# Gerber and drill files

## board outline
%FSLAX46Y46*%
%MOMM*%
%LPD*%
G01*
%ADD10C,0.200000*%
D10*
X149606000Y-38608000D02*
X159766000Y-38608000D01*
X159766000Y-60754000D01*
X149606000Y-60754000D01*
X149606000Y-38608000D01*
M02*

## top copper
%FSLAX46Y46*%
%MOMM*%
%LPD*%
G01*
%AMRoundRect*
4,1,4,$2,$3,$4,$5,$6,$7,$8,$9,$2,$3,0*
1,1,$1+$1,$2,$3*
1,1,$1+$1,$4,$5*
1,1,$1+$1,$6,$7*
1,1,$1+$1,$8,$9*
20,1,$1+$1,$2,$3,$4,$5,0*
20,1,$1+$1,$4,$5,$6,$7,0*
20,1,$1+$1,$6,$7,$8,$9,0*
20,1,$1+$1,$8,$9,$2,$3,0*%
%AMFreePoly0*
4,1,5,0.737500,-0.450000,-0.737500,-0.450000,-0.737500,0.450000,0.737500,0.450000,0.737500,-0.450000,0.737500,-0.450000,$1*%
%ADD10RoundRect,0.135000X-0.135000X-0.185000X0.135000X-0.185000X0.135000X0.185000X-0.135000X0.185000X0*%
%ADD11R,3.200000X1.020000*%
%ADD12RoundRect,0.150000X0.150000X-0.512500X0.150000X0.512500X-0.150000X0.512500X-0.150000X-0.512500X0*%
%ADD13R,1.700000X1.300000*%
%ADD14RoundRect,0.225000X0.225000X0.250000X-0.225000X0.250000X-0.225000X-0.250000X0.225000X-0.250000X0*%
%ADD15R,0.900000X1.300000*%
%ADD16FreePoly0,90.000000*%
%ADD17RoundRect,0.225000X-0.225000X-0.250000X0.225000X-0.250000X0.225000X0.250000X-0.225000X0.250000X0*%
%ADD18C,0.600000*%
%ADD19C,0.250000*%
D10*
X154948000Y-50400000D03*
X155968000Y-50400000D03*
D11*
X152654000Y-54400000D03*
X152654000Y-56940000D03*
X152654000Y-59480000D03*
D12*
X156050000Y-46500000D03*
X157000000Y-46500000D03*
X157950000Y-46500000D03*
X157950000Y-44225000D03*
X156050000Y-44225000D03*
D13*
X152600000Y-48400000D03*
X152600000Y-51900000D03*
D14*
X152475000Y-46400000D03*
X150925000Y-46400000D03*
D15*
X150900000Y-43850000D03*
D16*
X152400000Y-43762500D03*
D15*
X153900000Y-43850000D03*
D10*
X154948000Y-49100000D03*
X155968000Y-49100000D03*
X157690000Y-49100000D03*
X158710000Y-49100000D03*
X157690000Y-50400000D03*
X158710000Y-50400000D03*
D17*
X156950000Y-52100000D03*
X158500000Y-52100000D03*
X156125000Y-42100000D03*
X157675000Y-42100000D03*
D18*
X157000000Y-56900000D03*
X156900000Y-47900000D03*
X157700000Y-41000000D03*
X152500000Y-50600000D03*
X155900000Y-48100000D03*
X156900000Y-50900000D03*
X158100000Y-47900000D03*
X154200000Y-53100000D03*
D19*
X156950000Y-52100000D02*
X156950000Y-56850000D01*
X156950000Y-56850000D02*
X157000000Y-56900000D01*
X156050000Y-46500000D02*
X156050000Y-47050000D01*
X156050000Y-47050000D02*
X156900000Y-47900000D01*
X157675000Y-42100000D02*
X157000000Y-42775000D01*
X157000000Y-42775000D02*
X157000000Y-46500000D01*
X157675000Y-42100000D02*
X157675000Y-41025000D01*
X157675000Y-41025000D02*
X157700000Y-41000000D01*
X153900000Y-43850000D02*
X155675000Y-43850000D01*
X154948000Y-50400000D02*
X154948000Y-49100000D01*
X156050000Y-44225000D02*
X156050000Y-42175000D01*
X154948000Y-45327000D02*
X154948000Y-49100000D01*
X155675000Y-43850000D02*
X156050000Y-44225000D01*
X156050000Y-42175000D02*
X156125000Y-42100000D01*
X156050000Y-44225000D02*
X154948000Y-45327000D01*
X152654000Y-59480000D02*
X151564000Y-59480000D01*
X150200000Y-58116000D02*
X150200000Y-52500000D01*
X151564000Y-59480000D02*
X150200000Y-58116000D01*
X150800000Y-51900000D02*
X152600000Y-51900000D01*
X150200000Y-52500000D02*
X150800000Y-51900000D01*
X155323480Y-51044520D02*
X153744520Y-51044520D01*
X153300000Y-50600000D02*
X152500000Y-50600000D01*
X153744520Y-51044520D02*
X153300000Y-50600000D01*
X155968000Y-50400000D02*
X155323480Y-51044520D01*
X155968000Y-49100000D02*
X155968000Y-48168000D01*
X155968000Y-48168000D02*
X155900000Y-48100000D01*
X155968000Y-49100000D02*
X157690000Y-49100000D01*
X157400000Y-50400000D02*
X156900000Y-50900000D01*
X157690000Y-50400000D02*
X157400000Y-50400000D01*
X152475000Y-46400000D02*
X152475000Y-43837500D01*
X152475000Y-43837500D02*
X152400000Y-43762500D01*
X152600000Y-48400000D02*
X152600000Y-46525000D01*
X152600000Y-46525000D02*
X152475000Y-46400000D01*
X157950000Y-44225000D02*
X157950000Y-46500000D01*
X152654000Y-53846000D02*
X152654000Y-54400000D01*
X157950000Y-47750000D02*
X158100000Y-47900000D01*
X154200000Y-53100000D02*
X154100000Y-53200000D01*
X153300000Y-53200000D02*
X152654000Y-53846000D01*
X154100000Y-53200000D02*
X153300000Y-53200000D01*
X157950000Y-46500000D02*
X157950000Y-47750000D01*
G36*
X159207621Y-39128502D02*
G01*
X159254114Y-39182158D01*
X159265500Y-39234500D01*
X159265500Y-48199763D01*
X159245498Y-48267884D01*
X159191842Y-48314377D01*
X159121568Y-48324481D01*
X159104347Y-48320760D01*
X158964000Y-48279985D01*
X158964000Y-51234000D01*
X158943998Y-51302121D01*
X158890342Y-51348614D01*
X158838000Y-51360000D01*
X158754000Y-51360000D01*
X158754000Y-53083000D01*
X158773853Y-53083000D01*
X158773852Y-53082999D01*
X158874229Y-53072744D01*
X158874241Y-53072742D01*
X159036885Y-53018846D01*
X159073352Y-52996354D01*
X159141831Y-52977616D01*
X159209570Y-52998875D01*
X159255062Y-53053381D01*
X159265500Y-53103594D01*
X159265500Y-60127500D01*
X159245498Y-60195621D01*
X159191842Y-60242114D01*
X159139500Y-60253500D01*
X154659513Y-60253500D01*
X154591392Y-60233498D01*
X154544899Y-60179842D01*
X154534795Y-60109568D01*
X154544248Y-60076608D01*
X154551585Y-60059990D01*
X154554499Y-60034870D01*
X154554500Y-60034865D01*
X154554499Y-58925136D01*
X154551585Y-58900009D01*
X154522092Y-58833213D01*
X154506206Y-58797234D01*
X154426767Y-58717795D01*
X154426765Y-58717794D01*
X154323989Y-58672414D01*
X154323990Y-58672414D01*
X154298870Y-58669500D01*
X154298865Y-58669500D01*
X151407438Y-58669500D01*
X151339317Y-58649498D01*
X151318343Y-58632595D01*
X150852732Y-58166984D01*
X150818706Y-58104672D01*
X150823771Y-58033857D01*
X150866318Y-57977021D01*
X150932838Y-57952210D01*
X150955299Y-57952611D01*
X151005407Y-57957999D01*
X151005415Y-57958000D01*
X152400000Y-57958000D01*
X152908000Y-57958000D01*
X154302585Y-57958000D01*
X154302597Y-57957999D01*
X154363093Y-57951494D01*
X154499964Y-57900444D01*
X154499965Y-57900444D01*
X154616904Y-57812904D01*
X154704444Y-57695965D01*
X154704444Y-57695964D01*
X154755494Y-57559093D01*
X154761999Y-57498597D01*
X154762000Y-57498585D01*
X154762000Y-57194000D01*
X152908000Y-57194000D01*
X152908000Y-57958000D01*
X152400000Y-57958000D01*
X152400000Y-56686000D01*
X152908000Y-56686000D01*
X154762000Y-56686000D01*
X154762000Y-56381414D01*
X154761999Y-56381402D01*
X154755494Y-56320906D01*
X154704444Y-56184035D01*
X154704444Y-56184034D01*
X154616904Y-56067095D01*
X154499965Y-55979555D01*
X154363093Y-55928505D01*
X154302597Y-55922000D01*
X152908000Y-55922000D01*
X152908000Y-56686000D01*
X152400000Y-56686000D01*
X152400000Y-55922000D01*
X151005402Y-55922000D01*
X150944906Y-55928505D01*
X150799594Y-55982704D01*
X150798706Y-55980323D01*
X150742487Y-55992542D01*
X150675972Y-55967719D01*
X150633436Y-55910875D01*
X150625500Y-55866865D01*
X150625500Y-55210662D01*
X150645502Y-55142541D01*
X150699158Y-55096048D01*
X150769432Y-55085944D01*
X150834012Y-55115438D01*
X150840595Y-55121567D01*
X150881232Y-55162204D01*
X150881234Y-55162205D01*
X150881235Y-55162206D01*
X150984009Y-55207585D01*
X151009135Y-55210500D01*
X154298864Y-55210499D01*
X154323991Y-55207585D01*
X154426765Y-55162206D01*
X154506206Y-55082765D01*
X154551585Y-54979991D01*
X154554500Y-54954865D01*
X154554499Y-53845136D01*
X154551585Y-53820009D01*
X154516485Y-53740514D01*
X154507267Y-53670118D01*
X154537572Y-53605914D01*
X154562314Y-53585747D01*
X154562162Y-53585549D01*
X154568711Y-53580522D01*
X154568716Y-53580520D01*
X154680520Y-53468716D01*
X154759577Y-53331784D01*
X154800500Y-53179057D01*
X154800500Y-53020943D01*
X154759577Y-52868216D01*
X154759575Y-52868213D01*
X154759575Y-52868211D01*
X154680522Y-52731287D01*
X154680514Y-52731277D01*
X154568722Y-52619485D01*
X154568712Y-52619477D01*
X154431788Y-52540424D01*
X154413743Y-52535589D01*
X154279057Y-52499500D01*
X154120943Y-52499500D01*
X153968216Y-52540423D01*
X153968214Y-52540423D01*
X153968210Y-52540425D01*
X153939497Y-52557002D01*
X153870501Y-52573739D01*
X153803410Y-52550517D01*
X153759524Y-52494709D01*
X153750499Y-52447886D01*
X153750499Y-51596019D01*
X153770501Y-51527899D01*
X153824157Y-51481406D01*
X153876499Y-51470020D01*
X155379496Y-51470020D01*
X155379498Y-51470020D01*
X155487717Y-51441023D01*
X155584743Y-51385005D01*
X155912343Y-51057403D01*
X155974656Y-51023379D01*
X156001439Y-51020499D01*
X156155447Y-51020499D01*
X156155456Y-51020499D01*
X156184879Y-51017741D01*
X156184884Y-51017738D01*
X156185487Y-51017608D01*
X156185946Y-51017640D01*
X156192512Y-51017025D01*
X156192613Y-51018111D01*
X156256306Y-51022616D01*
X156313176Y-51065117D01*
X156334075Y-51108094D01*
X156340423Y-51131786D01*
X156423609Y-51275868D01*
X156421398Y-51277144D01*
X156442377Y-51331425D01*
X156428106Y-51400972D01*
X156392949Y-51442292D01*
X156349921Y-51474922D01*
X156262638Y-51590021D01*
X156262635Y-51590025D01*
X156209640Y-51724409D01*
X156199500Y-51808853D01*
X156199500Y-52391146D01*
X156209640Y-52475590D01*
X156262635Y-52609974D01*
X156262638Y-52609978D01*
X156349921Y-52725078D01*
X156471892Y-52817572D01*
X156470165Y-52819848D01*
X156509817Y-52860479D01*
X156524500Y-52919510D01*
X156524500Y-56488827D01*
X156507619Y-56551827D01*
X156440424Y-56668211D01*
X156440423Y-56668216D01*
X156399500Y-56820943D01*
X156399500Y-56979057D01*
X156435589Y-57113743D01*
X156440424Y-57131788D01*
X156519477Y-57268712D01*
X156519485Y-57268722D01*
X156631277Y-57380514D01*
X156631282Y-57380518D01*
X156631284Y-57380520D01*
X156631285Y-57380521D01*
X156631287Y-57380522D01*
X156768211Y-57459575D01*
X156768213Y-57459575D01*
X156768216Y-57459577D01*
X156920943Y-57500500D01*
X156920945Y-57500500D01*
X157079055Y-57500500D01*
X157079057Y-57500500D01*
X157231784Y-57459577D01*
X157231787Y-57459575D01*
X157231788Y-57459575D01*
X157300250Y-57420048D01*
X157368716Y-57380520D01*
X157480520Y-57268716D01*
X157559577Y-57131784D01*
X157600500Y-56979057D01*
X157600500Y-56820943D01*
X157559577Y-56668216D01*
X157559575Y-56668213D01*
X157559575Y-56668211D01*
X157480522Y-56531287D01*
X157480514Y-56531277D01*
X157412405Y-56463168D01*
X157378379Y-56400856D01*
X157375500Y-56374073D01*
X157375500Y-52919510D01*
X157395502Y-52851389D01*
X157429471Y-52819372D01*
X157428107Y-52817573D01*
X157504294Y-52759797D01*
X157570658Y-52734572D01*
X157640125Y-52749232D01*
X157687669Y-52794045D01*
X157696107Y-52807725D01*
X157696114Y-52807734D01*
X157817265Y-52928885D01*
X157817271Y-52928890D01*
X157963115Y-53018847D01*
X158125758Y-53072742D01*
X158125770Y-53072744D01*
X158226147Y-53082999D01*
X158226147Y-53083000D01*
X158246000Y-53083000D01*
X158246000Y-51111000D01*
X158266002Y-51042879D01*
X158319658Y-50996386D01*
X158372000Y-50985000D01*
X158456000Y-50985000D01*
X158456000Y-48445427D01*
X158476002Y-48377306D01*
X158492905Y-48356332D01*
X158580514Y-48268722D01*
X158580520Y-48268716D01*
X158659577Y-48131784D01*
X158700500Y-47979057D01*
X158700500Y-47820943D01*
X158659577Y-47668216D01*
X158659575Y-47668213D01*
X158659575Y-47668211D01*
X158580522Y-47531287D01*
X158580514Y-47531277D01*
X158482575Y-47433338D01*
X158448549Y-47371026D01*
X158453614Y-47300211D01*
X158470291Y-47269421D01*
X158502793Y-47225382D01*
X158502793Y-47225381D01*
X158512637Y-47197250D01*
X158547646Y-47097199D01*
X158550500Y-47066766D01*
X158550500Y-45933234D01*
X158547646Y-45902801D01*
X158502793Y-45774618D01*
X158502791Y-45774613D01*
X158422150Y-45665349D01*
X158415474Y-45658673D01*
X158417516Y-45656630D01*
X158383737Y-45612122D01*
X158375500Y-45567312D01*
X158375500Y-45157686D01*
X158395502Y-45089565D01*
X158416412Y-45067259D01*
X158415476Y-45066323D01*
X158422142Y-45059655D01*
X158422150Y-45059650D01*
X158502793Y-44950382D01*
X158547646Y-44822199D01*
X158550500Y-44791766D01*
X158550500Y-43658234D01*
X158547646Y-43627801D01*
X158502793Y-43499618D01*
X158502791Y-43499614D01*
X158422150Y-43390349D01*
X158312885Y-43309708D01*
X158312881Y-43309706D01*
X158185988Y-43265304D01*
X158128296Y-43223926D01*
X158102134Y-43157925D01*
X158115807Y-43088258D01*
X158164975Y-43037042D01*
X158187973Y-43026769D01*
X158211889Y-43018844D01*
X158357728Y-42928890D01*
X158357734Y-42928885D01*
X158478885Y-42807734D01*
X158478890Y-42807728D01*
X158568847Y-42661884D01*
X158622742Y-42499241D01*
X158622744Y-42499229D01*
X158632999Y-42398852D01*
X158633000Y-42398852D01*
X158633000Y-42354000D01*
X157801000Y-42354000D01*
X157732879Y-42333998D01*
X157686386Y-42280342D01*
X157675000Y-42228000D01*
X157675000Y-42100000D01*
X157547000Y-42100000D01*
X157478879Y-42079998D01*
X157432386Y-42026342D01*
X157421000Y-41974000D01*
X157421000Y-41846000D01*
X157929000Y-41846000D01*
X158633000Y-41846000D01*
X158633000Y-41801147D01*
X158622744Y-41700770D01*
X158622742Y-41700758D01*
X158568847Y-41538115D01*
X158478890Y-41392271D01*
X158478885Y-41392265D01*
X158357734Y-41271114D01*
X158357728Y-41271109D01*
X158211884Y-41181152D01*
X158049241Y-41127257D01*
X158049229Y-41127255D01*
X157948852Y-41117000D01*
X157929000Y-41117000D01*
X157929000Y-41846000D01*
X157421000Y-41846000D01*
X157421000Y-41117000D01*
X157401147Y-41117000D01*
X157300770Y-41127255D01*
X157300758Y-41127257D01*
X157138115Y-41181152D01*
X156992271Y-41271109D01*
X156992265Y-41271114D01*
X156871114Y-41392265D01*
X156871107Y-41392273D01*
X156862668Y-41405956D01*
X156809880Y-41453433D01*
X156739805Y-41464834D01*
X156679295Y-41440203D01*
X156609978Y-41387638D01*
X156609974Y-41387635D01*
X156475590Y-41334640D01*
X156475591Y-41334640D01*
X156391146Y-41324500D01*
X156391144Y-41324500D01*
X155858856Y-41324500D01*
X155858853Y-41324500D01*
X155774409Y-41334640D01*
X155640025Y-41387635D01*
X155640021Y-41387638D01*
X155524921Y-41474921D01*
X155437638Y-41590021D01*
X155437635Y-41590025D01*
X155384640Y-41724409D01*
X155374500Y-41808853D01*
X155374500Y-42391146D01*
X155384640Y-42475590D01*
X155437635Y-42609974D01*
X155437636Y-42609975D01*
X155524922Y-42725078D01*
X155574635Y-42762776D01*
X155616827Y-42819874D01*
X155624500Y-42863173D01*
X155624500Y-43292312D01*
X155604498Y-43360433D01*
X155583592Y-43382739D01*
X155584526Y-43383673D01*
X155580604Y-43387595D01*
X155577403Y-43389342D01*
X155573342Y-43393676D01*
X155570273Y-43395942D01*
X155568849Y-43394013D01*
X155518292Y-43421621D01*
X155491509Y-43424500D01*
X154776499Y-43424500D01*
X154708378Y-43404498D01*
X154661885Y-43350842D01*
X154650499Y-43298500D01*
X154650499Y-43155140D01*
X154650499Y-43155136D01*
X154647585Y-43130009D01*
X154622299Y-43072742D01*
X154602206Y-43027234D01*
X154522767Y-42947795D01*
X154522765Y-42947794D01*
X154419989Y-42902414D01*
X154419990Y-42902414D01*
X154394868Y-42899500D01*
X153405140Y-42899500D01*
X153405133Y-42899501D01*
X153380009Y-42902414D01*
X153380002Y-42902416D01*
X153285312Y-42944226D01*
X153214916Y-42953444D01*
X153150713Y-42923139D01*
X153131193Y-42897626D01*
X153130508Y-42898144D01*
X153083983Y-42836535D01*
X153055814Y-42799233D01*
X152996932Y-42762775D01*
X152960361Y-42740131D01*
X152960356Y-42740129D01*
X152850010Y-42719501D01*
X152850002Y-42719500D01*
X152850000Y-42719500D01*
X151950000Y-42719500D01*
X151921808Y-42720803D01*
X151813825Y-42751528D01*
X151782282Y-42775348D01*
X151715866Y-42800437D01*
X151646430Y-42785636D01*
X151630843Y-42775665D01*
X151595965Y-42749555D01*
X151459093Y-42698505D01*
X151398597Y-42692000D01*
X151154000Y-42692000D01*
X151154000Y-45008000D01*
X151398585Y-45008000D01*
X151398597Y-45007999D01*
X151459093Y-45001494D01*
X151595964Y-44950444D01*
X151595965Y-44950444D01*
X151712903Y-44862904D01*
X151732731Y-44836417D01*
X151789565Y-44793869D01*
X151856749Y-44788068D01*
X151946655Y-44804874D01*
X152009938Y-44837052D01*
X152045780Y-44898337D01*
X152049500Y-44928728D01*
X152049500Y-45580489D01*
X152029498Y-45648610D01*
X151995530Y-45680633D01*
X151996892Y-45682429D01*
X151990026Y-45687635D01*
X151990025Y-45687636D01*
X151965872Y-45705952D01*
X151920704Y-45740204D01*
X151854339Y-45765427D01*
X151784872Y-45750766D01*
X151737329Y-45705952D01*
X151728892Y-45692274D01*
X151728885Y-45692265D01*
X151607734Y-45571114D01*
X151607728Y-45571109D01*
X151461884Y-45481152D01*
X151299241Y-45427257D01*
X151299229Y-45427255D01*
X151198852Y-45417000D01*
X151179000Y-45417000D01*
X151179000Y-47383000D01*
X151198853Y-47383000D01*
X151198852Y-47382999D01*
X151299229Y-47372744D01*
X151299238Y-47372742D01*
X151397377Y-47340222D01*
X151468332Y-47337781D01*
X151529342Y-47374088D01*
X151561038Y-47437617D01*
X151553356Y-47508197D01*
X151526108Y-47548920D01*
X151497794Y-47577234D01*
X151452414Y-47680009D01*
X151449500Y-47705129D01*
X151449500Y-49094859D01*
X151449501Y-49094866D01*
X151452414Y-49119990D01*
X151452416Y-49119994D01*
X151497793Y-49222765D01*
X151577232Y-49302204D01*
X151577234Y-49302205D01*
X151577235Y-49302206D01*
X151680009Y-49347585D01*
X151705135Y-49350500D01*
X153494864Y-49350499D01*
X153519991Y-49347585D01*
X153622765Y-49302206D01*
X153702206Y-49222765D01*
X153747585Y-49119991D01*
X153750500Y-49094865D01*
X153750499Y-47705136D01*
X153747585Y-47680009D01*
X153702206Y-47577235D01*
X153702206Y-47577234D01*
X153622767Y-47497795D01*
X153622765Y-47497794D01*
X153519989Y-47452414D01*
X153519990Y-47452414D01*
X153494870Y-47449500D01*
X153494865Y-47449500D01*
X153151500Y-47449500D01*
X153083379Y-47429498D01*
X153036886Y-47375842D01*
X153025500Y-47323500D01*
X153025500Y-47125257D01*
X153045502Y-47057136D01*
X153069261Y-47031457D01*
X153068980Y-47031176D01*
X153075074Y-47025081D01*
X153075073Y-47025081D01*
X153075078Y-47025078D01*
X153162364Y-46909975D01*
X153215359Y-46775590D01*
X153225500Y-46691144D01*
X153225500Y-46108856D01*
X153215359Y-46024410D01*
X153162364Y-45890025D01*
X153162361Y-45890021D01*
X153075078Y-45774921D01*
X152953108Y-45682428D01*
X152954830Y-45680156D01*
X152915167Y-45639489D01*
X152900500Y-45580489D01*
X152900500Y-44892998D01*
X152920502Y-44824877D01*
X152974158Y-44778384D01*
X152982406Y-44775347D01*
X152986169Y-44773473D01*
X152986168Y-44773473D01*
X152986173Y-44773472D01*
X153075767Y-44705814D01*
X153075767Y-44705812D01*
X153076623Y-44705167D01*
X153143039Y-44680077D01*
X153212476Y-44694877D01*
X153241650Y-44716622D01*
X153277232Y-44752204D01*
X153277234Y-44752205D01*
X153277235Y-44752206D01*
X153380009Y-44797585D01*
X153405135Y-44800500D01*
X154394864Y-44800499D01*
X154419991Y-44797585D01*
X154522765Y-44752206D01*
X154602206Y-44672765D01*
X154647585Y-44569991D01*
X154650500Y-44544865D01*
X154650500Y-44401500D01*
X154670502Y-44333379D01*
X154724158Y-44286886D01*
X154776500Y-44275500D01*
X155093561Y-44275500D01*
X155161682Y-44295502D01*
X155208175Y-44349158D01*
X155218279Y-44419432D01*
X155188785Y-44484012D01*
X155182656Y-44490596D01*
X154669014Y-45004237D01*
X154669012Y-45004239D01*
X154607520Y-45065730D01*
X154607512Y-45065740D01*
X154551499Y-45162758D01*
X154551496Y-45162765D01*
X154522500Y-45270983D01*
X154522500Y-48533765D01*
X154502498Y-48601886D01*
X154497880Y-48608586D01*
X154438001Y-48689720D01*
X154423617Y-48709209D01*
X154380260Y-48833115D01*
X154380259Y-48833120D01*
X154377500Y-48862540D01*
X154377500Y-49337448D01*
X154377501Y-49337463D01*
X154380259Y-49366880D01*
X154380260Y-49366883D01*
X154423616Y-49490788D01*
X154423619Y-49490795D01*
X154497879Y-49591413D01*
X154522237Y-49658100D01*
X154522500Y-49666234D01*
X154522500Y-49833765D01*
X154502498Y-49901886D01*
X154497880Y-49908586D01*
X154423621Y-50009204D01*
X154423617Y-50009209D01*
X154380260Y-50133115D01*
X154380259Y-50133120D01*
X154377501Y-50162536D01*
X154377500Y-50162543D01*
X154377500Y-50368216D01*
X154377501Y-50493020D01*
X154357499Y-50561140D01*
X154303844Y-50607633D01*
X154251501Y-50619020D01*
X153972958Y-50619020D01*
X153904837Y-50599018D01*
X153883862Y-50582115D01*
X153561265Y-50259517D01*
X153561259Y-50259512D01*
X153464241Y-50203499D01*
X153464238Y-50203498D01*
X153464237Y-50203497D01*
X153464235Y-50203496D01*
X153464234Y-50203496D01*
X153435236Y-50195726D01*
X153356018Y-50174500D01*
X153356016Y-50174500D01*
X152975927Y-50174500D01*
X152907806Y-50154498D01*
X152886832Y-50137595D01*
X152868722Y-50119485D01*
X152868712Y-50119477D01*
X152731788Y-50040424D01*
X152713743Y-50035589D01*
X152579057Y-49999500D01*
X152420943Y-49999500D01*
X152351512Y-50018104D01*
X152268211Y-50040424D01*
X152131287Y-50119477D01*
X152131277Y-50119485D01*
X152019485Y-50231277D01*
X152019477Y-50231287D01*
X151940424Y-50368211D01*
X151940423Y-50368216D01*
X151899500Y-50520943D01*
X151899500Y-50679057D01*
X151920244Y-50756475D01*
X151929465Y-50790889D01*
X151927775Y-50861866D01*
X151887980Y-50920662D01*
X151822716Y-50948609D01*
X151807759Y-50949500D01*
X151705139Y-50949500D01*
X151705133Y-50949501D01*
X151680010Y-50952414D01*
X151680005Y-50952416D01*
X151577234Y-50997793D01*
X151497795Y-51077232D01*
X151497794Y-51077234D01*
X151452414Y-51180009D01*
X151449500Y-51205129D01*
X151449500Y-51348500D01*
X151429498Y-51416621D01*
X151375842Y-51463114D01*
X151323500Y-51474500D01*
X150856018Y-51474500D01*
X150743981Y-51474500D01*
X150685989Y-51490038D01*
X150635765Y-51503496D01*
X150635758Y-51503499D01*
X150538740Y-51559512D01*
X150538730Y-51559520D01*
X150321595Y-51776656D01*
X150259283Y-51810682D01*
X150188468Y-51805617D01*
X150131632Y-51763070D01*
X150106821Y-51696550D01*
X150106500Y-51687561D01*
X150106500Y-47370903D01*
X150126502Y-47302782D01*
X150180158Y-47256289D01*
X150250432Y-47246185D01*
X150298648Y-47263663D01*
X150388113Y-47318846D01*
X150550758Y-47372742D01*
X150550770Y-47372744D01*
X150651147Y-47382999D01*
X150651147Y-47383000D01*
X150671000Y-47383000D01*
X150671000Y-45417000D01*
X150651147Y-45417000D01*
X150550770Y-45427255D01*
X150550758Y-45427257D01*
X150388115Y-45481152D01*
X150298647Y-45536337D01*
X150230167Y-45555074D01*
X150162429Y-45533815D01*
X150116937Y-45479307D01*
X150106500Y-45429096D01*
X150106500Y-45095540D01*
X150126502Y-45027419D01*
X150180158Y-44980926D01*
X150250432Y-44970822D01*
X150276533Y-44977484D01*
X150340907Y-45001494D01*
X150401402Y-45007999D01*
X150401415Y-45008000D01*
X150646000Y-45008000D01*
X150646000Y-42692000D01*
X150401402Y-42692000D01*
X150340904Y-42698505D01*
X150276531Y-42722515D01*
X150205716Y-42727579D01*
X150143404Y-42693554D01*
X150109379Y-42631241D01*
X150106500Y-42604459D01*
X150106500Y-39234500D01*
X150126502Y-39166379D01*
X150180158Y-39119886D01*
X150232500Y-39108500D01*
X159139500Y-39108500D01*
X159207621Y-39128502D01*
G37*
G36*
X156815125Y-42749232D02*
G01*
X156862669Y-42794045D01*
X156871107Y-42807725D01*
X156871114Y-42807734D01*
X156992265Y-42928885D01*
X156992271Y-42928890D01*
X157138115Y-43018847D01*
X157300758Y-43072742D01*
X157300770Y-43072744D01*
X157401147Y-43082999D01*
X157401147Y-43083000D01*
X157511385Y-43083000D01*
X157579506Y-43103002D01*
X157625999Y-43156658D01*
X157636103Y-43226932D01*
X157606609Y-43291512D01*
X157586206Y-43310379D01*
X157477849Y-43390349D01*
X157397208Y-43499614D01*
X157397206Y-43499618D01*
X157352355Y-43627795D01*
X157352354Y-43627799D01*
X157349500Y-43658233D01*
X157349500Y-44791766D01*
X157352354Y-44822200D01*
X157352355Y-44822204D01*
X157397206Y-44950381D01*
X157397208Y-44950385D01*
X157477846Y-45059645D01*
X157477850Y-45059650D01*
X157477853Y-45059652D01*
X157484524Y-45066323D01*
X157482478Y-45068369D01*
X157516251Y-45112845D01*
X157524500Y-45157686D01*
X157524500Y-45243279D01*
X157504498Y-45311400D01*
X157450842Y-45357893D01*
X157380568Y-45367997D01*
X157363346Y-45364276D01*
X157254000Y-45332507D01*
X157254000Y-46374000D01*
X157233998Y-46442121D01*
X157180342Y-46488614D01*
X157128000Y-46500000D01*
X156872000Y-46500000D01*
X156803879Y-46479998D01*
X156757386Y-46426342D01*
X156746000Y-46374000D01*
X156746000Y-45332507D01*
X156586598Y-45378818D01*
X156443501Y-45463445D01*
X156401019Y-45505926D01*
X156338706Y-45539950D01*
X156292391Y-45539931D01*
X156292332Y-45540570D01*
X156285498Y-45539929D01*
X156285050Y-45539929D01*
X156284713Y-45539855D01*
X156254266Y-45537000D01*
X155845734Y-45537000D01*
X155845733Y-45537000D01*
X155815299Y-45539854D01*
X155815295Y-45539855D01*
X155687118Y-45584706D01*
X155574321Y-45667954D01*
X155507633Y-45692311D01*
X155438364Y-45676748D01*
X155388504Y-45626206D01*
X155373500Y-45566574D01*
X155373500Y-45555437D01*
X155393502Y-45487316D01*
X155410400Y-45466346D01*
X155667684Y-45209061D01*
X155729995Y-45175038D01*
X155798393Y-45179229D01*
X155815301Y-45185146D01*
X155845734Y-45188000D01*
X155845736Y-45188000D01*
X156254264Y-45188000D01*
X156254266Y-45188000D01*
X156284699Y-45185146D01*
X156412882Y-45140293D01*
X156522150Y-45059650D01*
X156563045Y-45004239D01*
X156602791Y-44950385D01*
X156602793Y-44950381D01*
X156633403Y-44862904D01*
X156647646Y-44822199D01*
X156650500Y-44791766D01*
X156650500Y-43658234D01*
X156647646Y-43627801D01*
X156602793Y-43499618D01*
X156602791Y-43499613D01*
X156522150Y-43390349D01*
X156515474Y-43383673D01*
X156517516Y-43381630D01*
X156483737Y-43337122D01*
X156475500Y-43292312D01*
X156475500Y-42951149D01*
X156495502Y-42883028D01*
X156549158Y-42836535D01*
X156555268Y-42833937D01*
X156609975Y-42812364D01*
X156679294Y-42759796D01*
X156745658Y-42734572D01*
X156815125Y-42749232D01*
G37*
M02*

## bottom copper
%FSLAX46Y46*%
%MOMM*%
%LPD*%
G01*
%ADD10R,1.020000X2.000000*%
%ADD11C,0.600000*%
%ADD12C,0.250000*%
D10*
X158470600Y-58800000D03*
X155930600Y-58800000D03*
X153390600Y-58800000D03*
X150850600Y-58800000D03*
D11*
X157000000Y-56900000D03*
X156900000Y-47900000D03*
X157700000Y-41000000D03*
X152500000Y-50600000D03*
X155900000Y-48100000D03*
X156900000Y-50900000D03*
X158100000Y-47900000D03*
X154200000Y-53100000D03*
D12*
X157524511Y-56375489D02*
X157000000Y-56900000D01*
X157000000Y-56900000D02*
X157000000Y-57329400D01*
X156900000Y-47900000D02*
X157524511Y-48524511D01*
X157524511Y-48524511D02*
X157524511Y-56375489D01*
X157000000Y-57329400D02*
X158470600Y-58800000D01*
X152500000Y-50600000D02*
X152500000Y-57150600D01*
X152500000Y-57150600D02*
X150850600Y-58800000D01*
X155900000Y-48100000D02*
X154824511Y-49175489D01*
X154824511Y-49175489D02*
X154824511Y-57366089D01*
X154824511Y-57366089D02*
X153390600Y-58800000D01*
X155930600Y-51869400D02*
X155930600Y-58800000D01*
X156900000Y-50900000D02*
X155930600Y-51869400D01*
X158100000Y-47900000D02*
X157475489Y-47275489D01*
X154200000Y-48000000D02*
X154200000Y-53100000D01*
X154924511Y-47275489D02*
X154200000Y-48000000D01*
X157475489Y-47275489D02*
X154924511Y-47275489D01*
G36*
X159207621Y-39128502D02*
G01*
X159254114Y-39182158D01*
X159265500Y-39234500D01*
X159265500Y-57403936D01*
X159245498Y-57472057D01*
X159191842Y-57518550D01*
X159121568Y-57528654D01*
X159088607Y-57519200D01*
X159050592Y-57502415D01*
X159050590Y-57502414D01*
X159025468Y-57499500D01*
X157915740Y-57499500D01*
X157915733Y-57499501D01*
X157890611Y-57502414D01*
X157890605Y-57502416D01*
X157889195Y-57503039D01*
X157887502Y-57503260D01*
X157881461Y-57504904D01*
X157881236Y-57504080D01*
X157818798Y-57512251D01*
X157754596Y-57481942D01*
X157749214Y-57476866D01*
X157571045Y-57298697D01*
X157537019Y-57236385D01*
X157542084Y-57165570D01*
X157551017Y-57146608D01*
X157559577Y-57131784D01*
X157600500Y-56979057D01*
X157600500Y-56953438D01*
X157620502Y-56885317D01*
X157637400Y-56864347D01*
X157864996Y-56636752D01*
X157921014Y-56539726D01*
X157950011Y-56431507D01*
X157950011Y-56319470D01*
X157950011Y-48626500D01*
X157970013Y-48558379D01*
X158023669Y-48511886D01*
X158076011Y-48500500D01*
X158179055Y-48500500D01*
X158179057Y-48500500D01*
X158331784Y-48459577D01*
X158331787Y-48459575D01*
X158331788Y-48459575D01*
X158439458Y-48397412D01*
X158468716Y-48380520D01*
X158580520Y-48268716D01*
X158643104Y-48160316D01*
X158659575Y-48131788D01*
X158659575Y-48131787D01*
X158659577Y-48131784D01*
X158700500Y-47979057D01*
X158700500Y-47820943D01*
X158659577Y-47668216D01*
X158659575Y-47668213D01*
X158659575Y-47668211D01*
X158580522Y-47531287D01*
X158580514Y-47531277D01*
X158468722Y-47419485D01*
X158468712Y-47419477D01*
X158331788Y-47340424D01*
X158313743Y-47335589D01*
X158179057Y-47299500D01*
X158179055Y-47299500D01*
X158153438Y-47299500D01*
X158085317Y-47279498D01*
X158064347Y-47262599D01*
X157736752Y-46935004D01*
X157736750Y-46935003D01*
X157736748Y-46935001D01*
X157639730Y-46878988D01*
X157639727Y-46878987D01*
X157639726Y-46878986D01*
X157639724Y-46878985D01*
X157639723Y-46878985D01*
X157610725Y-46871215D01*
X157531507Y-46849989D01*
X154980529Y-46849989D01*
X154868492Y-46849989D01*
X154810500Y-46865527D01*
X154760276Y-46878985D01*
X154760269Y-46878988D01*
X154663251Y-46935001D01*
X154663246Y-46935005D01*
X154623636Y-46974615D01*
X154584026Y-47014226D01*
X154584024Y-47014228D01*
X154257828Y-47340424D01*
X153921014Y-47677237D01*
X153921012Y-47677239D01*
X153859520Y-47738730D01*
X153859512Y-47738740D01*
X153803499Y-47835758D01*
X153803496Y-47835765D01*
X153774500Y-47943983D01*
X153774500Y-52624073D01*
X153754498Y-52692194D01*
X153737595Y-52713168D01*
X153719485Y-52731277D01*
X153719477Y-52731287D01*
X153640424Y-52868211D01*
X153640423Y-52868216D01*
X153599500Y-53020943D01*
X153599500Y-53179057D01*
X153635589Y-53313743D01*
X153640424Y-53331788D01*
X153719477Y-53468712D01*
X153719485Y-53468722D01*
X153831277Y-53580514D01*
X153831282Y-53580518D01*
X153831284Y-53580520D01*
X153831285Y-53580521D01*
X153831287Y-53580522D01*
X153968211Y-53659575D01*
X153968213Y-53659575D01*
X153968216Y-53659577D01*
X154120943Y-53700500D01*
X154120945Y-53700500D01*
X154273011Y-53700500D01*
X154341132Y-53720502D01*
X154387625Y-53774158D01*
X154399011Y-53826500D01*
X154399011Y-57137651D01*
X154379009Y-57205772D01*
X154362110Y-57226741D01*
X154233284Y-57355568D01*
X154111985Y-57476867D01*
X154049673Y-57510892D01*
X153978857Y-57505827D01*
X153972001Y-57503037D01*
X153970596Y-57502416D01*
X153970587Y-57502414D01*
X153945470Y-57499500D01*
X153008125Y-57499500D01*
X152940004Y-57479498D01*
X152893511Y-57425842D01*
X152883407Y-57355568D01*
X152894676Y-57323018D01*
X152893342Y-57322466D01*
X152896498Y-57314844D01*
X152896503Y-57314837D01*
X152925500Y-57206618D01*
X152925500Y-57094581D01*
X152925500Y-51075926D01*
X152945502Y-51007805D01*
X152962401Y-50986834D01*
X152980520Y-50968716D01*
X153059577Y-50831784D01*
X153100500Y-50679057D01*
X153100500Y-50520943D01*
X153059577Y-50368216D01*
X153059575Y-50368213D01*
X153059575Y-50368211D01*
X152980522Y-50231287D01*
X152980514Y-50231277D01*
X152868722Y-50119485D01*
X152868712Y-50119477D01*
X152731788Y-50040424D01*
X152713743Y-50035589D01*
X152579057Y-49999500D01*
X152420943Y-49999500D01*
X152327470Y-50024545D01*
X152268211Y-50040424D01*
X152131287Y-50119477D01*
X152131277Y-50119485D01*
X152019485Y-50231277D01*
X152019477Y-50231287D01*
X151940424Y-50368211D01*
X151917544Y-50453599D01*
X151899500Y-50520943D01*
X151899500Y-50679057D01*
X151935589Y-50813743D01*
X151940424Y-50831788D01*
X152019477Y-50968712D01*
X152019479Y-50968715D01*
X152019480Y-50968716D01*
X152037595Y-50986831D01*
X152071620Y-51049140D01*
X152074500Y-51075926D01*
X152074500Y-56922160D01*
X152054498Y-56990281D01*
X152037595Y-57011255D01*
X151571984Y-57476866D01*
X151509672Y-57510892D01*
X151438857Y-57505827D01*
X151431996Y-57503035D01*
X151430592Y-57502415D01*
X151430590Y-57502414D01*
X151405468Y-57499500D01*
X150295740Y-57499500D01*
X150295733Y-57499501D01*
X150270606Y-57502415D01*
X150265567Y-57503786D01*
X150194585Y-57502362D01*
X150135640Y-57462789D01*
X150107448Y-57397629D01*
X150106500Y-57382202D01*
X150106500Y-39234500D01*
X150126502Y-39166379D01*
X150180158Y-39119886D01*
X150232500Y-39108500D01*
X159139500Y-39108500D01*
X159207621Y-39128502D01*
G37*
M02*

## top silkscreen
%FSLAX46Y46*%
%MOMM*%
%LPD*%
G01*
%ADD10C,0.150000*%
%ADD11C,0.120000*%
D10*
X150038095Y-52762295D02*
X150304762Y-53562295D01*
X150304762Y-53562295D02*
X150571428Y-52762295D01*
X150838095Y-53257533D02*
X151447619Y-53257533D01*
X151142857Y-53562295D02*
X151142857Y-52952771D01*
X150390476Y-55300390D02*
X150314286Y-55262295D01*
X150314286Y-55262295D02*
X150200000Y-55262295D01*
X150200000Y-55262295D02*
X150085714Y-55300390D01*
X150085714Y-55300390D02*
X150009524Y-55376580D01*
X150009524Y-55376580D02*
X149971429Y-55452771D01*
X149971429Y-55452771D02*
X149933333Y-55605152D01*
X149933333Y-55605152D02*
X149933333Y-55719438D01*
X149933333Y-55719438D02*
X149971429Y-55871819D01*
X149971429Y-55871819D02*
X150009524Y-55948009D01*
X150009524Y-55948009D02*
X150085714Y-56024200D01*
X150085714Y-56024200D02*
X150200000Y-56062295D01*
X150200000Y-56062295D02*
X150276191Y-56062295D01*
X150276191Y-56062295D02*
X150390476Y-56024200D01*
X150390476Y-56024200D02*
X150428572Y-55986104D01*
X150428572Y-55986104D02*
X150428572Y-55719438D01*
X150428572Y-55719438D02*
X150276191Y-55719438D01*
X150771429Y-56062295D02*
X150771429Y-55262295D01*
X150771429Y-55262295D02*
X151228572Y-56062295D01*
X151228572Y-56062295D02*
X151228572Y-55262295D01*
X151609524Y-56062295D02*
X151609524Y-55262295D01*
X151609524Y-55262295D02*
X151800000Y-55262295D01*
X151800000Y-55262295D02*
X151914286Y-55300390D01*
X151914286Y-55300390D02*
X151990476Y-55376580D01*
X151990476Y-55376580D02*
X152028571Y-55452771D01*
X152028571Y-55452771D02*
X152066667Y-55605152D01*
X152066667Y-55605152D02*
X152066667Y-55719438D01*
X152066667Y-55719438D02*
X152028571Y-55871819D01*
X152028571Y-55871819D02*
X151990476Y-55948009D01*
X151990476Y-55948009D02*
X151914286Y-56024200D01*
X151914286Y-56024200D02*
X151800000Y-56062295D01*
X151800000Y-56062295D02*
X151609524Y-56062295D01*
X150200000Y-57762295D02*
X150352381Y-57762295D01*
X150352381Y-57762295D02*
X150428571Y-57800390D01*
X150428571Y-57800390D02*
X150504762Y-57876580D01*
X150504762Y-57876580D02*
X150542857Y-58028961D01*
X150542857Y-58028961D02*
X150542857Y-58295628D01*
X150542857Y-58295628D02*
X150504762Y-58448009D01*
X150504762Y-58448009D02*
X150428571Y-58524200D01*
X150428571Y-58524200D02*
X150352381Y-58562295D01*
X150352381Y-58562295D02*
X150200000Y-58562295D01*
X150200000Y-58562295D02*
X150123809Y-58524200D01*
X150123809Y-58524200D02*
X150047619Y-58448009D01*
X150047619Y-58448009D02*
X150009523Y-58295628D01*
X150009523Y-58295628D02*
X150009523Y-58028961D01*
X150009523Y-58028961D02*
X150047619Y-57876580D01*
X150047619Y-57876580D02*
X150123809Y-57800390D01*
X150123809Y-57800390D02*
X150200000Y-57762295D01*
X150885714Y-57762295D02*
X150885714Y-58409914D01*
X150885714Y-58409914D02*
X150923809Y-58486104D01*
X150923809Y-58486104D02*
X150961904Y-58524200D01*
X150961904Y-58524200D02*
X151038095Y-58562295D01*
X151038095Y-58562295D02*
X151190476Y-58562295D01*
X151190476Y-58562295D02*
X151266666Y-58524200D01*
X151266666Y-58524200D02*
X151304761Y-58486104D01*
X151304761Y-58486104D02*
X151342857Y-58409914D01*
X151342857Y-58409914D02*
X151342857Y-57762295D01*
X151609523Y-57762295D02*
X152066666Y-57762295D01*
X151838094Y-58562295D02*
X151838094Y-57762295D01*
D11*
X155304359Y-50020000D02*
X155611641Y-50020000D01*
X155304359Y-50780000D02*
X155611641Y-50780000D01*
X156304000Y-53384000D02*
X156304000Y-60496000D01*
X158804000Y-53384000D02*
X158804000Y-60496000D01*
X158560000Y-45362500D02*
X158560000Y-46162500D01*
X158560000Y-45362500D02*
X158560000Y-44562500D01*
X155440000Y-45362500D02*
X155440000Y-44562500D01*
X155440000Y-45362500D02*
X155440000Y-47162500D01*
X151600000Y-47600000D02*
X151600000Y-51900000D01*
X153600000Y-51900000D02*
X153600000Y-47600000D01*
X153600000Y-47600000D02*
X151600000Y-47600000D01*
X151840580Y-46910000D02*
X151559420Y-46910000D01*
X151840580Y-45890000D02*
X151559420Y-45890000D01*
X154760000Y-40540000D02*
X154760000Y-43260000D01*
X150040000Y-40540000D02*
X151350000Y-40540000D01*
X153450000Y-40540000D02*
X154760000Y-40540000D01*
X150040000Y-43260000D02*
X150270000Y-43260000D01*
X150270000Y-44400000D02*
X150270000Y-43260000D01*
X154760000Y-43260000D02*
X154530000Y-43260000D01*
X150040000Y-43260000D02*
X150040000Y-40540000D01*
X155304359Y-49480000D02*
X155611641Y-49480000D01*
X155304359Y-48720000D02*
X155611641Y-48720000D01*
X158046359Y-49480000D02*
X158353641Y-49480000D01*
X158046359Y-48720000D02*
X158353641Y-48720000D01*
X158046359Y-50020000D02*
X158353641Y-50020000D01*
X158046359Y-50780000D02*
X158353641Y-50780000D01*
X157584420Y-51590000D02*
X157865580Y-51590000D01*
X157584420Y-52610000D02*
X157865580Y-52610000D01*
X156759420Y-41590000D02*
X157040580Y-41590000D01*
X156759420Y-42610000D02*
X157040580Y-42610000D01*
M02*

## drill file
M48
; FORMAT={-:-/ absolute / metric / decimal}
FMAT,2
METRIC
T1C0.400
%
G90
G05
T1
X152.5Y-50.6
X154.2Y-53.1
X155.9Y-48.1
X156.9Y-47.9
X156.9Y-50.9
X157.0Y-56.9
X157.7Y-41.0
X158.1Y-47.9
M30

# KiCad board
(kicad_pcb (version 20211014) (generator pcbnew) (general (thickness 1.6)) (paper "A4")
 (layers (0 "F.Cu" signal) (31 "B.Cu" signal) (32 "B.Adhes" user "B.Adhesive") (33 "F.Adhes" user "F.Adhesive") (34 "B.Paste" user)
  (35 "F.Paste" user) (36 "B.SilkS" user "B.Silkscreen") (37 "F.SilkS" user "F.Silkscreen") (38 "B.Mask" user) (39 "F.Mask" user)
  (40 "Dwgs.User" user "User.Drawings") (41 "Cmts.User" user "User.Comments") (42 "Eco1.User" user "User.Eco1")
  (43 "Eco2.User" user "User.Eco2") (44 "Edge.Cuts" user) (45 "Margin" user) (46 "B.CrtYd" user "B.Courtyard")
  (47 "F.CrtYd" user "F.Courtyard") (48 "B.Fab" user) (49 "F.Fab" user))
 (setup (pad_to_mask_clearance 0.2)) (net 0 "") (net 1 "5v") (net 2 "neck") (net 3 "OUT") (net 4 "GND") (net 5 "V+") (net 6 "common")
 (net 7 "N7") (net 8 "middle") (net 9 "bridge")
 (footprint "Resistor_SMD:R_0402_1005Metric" (layer "F.Cu") (at 155.458 50.4)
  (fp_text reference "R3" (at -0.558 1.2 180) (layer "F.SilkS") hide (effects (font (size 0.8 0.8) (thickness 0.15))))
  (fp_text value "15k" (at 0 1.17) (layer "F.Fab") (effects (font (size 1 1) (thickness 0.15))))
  (fp_line (start -0.153641 -0.38) (end 0.153641 -0.38) (layer "F.SilkS") (width 0.12))
  (fp_line (start -0.153641 0.38) (end 0.153641 0.38) (layer "F.SilkS") (width 0.12))
  (pad "1" smd roundrect (at -0.51 0) (size 0.54 0.64) (layers "F.Cu" "F.Paste" "F.Mask") (roundrect_rratio 0.25) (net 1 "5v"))
  (pad "2" smd roundrect (at 0.51 0) (size 0.54 0.64) (layers "F.Cu" "F.Paste" "F.Mask") (roundrect_rratio 0.25) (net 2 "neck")))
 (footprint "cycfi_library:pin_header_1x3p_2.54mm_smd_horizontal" (layer "F.Cu") (at 152.654 54.4)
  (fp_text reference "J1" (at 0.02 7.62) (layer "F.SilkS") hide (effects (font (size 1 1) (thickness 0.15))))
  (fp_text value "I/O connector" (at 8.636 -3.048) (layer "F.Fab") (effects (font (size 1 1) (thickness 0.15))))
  (fp_line (start 3.65 -1.016) (end 3.65 6.096) (layer "F.SilkS") (width 0.12))
  (fp_line (start 6.15 -1.016) (end 6.15 6.096) (layer "F.SilkS") (width 0.12))
  (pad "1" smd rect (at 0 0) (size 3.2 1.02) (layers "F.Cu" "F.Paste" "F.Mask") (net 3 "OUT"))
  (pad "2" smd rect (at 0 2.54) (size 3.2 1.02) (layers "F.Cu" "F.Paste" "F.Mask") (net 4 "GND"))
  (pad "3" smd rect (at 0 5.08) (size 3.2 1.02) (layers "F.Cu" "F.Paste" "F.Mask") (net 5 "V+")))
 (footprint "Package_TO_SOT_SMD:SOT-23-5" (layer "F.Cu") (at 157 45.3625 90)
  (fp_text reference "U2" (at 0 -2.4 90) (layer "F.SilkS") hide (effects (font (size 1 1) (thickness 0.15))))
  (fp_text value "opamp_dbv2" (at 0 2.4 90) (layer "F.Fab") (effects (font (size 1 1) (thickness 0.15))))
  (fp_line (start 0 1.56) (end -0.8 1.56) (layer "F.SilkS") (width 0.12))
  (fp_line (start 0 1.56) (end 0.8 1.56) (layer "F.SilkS") (width 0.12))
  (fp_line (start 0 -1.56) (end 0.8 -1.56) (layer "F.SilkS") (width 0.12))
  (fp_line (start 0 -1.56) (end -1.8 -1.56) (layer "F.SilkS") (width 0.12))
  (pad "1" smd roundrect (at -1.1375 -0.95 90) (size 1.325 0.6) (layers "F.Cu" "F.Paste" "F.Mask") (roundrect_rratio 0.25) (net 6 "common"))
  (pad "2" smd roundrect (at -1.1375 0 90) (size 1.325 0.6) (layers "F.Cu" "F.Paste" "F.Mask") (roundrect_rratio 0.25) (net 4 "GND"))
  (pad "3" smd roundrect (at -1.1375 0.95 90) (size 1.325 0.6) (layers "F.Cu" "F.Paste" "F.Mask") (roundrect_rratio 0.25) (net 3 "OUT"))
  (pad "4" smd roundrect (at 1.1375 0.95 90) (size 1.325 0.6) (layers "F.Cu" "F.Paste" "F.Mask") (roundrect_rratio 0.25) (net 3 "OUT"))
  (pad "5" smd roundrect (at 1.1375 -0.95 90) (size 1.325 0.6) (layers "F.Cu" "F.Paste" "F.Mask") (roundrect_rratio 0.25) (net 1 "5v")))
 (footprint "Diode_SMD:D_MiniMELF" (layer "F.Cu") (at 152.6 50.15 -90)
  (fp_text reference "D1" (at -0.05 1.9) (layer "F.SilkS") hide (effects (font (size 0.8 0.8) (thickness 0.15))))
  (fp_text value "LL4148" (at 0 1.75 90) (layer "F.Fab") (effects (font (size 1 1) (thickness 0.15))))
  (fp_line (start -2.55 1) (end 1.75 1) (layer "F.SilkS") (width 0.12))
  (fp_line (start 1.75 -1) (end -2.55 -1) (layer "F.SilkS") (width 0.12))
  (fp_line (start -2.55 -1) (end -2.55 1) (layer "F.SilkS") (width 0.12))
  (pad "1" smd rect (at -1.75 0 270) (size 1.3 1.7) (layers "F.Cu" "F.Paste" "F.Mask") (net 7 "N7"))
  (pad "2" smd rect (at 1.75 0 270) (size 1.3 1.7) (layers "F.Cu" "F.Paste" "F.Mask") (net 5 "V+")))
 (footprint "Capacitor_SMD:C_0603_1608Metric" (layer "F.Cu") (at 151.7 46.4 180)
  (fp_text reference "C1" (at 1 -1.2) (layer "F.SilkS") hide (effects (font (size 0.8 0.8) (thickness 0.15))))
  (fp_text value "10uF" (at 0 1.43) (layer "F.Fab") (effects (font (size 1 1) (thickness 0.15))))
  (fp_line (start -0.14058 -0.51) (end 0.14058 -0.51) (layer "F.SilkS") (width 0.12))
  (fp_line (start -0.14058 0.51) (end 0.14058 0.51) (layer "F.SilkS") (width 0.12))
  (pad "1" smd roundrect (at -0.775 0 180) (size 0.9 0.95) (layers "F.Cu" "F.Paste" "F.Mask") (roundrect_rratio 0.25) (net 7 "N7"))
  (pad "2" smd roundrect (at 0.775 0 180) (size 0.9 0.95) (layers "F.Cu" "F.Paste" "F.Mask") (roundrect_rratio 0.25) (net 4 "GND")))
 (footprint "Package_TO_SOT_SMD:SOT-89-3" (layer "F.Cu") (at 152.4 42.2 90)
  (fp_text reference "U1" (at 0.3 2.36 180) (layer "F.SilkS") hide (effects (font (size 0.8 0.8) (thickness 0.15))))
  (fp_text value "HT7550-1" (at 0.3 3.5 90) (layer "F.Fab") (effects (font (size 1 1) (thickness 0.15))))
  (fp_line (start 1.66 2.36) (end -1.06 2.36) (layer "F.SilkS") (width 0.12))
  (fp_line (start 1.66 -2.36) (end 1.66 -1.05) (layer "F.SilkS") (width 0.12))
  (fp_line (start 1.66 1.05) (end 1.66 2.36) (layer "F.SilkS") (width 0.12))
  (fp_line (start -1.06 -2.36) (end -1.06 -2.13) (layer "F.SilkS") (width 0.12))
  (fp_line (start -2.2 -2.13) (end -1.06 -2.13) (layer "F.SilkS") (width 0.12))
  (fp_line (start -1.06 2.36) (end -1.06 2.13) (layer "F.SilkS") (width 0.12))
  (fp_line (start -1.06 -2.36) (end 1.66 -2.36) (layer "F.SilkS") (width 0.12))
  (pad "1" smd rect (at -1.65 -1.5 90) (size 1.3 0.9) (layers "F.Cu" "F.Paste" "F.Mask") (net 4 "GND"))
  (pad "2" smd custom (at -1.5625 0 90) (size 1.475 0.9) (layers "F.Cu" "F.Paste" "F.Mask") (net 7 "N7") (zone_connect 2)
   (options (clearance outline) (anchor rect)) (primitives))
  (pad "3" smd rect (at -1.65 1.5 90) (size 1.3 0.9) (layers "F.Cu" "F.Paste" "F.Mask") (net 1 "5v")))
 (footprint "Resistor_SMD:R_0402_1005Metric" (layer "F.Cu") (at 155.458 49.1)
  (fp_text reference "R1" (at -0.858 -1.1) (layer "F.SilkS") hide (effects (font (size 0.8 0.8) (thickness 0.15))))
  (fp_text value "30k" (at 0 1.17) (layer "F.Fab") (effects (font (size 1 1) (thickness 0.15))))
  (fp_line (start -0.153641 0.38) (end 0.153641 0.38) (layer "F.SilkS") (width 0.12))
  (fp_line (start -0.153641 -0.38) (end 0.153641 -0.38) (layer "F.SilkS") (width 0.12))
  (pad "1" smd roundrect (at -0.51 0) (size 0.54 0.64) (layers "F.Cu" "F.Paste" "F.Mask") (roundrect_rratio 0.25) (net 1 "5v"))
  (pad "2" smd roundrect (at 0.51 0) (size 0.54 0.64) (layers "F.Cu" "F.Paste" "F.Mask") (roundrect_rratio 0.25) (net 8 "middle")))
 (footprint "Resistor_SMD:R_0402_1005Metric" (layer "F.Cu") (at 158.2 49.1)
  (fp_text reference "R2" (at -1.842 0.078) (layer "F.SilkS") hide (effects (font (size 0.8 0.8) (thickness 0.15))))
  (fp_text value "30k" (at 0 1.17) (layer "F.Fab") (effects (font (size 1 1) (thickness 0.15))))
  (fp_line (start -0.153641 0.38) (end 0.153641 0.38) (layer "F.SilkS") (width 0.12))
  (fp_line (start -0.153641 -0.38) (end 0.153641 -0.38) (layer "F.SilkS") (width 0.12))
  (pad "1" smd roundrect (at -0.51 0) (size 0.54 0.64) (layers "F.Cu" "F.Paste" "F.Mask") (roundrect_rratio 0.25) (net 8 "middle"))
  (pad "2" smd roundrect (at 0.51 0) (size 0.54 0.64) (layers "F.Cu" "F.Paste" "F.Mask") (roundrect_rratio 0.25) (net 4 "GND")))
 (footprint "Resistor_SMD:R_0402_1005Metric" (layer "F.Cu") (at 158.2 50.4)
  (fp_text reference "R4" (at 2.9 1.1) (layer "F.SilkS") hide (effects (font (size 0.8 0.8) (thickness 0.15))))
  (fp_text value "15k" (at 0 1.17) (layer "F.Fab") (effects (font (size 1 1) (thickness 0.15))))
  (fp_line (start -0.153641 -0.38) (end 0.153641 -0.38) (layer "F.SilkS") (width 0.12))
  (fp_line (start -0.153641 0.38) (end 0.153641 0.38) (layer "F.SilkS") (width 0.12))
  (pad "1" smd roundrect (at -0.51 0) (size 0.54 0.64) (layers "F.Cu" "F.Paste" "F.Mask") (roundrect_rratio 0.25) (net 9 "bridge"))
  (pad "2" smd roundrect (at 0.51 0) (size 0.54 0.64) (layers "F.Cu" "F.Paste" "F.Mask") (roundrect_rratio 0.25) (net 4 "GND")))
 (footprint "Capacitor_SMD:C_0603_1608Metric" (layer "F.Cu") (at 157.725 52.1)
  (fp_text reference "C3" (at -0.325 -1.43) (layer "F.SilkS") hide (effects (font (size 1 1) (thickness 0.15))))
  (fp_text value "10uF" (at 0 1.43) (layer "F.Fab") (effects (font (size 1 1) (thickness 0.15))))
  (fp_line (start -0.14058 -0.51) (end 0.14058 -0.51) (layer "F.SilkS") (width 0.12))
  (fp_line (start -0.14058 0.51) (end 0.14058 0.51) (layer "F.SilkS") (width 0.12))
  (pad "1" smd roundrect (at -0.775 0) (size 0.9 0.95) (layers "F.Cu" "F.Paste" "F.Mask") (roundrect_rratio 0.25) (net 6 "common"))
  (pad "2" smd roundrect (at 0.775 0) (size 0.9 0.95) (layers "F.Cu" "F.Paste" "F.Mask") (roundrect_rratio 0.25) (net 4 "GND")))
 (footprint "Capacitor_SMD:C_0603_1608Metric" (layer "F.Cu") (at 156.9 42.1)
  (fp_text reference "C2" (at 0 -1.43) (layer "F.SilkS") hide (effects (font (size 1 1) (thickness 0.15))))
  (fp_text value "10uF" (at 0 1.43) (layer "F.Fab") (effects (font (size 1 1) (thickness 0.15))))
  (fp_line (start -0.14058 -0.51) (end 0.14058 -0.51) (layer "F.SilkS") (width 0.12))
  (fp_line (start -0.14058 0.51) (end 0.14058 0.51) (layer "F.SilkS") (width 0.12))
  (pad "1" smd roundrect (at -0.775 0) (size 0.9 0.95) (layers "F.Cu" "F.Paste" "F.Mask") (roundrect_rratio 0.25) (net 1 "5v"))
  (pad "2" smd roundrect (at 0.775 0) (size 0.9 0.95) (layers "F.Cu" "F.Paste" "F.Mask") (roundrect_rratio 0.25) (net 4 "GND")))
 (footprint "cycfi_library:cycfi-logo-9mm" (layer "B.Cu") (at 154.7 39.8 180)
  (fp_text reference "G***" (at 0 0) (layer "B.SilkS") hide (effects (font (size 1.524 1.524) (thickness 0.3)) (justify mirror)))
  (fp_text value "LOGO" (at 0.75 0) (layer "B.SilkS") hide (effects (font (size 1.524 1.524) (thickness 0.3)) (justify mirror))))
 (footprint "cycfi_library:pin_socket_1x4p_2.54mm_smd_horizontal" (layer "B.Cu") (at 158.4706 58.8 90)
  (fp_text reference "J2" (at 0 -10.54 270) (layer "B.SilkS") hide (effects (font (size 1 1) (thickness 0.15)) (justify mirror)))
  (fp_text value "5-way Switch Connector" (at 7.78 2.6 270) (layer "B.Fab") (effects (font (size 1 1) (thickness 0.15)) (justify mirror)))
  (pad "1" smd rect (at 0 0 90) (size 2 1.02) (layers "B.Cu" "B.Paste" "B.Mask") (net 6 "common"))
  (pad "2" smd rect (at 0 -2.54 90) (size 2 1.02) (layers "B.Cu" "B.Paste" "B.Mask") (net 9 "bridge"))
  (pad "3" smd rect (at 0 -5.08 90) (size 2 1.02) (layers "B.Cu" "B.Paste" "B.Mask") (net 8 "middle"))
  (pad "4" smd rect (at 0 -7.62 90) (size 2 1.02) (layers "B.Cu" "B.Paste" "B.Mask") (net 2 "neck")))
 (gr_rect (start 149.606 38.608) (end 159.766 60.754) (layer "Edge.Cuts") (width 0.2) (fill none))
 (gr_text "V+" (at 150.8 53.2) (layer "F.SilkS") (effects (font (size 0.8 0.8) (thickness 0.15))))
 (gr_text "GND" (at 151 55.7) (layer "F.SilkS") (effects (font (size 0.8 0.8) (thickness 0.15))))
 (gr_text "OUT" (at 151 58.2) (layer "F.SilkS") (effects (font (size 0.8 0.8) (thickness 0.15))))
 (segment (start 156.95 52.1) (end 156.95 56.85) (width 0.25) (layer "F.Cu") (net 6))
 (segment (start 156.95 56.85) (end 157 56.9) (width 0.25) (layer "F.Cu") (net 6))
 (segment (start 156.05 46.5) (end 156.05 47.05) (width 0.25) (layer "F.Cu") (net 6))
 (segment (start 156.05 47.05) (end 156.9 47.9) (width 0.25) (layer "F.Cu") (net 6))
 (via (at 157 56.9) (size 0.6) (drill 0.4) (layers "F.Cu" "B.Cu") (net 6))
 (via (at 156.9 47.9) (size 0.6) (drill 0.4) (layers "F.Cu" "B.Cu") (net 6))
 (segment (start 157.524511 56.375489) (end 157 56.9) (width 0.25) (layer "B.Cu") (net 6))
 (segment (start 157 56.9) (end 157 57.3294) (width 0.25) (layer "B.Cu") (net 6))
 (segment (start 156.9 47.9) (end 157.524511 48.524511) (width 0.25) (layer "B.Cu") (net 6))
 (segment (start 157.524511 48.524511) (end 157.524511 56.375489) (width 0.25) (layer "B.Cu") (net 6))
 (segment (start 157 57.3294) (end 158.4706 58.8) (width 0.25) (layer "B.Cu") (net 6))
 (segment (start 157.675 42.1) (end 157 42.775) (width 0.25) (layer "F.Cu") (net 4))
 (segment (start 157 42.775) (end 157 46.5) (width 0.25) (layer "F.Cu") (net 4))
 (segment (start 157.675 42.1) (end 157.675 41.025) (width 0.25) (layer "F.Cu") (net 4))
 (segment (start 157.675 41.025) (end 157.7 41) (width 0.25) (layer "F.Cu") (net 4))
 (via (at 157.7 41) (size 0.6) (drill 0.4) (layers "F.Cu" "B.Cu") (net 4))
 (segment (start 153.9 43.85) (end 155.675 43.85) (width 0.25) (layer "F.Cu") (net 1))
 (segment (start 154.948 50.4) (end 154.948 49.1) (width 0.25) (layer "F.Cu") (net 1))
 (segment (start 156.05 44.225) (end 156.05 42.175) (width 0.25) (layer "F.Cu") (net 1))
 (segment (start 154.948 45.327) (end 154.948 49.1) (width 0.25) (layer "F.Cu") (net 1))
 (segment (start 155.675 43.85) (end 156.05 44.225) (width 0.25) (layer "F.Cu") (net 1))
 (segment (start 156.05 42.175) (end 156.125 42.1) (width 0.25) (layer "F.Cu") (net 1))
 (segment (start 156.05 44.225) (end 154.948 45.327) (width 0.25) (layer "F.Cu") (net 1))
 (segment (start 152.654 59.48) (end 151.564 59.48) (width 0.25) (layer "F.Cu") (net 5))
 (segment (start 150.2 58.116) (end 150.2 52.5) (width 0.25) (layer "F.Cu") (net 5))
 (segment (start 151.564 59.48) (end 150.2 58.116) (width 0.25) (layer "F.Cu") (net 5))
 (segment (start 150.8 51.9) (end 152.6 51.9) (width 0.25) (layer "F.Cu") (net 5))
 (segment (start 150.2 52.5) (end 150.8 51.9) (width 0.25) (layer "F.Cu") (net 5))
 (segment (start 155.32348 51.04452) (end 153.74452 51.04452) (width 0.25) (layer "F.Cu") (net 2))
 (segment (start 153.3 50.6) (end 152.5 50.6) (width 0.25) (layer "F.Cu") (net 2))
 (segment (start 153.74452 51.04452) (end 153.3 50.6) (width 0.25) (layer "F.Cu") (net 2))
 (segment (start 155.968 50.4) (end 155.32348 51.04452) (width 0.25) (layer "F.Cu") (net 2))
 (via (at 152.5 50.6) (size 0.6) (drill 0.4) (layers "F.Cu" "B.Cu") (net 2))
 (segment (start 152.5 50.6) (end 152.5 57.1506) (width 0.25) (layer "B.Cu") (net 2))
 (segment (start 152.5 57.1506) (end 150.8506 58.8) (width 0.25) (layer "B.Cu") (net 2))
 (segment (start 155.968 49.1) (end 155.968 48.168) (width 0.25) (layer "F.Cu") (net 8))
 (segment (start 155.968 48.168) (end 155.9 48.1) (width 0.25) (layer "F.Cu") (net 8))
 (segment (start 155.968 49.1) (end 157.69 49.1) (width 0.25) (layer "F.Cu") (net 8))
 (via (at 155.9 48.1) (size 0.6) (drill 0.4) (layers "F.Cu" "B.Cu") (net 8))
 (segment (start 155.9 48.1) (end 154.824511 49.175489) (width 0.25) (layer "B.Cu") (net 8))
 (segment (start 154.824511 49.175489) (end 154.824511 57.366089) (width 0.25) (layer "B.Cu") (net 8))
 (segment (start 154.824511 57.366089) (end 153.3906 58.8) (width 0.25) (layer "B.Cu") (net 8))
 (segment (start 157.4 50.4) (end 156.9 50.9) (width 0.25) (layer "F.Cu") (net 9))
 (segment (start 157.69 50.4) (end 157.4 50.4) (width 0.25) (layer "F.Cu") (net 9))
 (via (at 156.9 50.9) (size 0.6) (drill 0.4) (layers "F.Cu" "B.Cu") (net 9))
 (segment (start 155.9306 51.8694) (end 155.9306 58.8) (width 0.25) (layer "B.Cu") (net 9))
 (segment (start 156.9 50.9) (end 155.9306 51.8694) (width 0.25) (layer "B.Cu") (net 9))
 (segment (start 152.475 46.4) (end 152.475 43.8375) (width 0.25) (layer "F.Cu") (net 7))
 (segment (start 152.475 43.8375) (end 152.4 43.7625) (width 0.25) (layer "F.Cu") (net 7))
 (segment (start 152.6 48.4) (end 152.6 46.525) (width 0.25) (layer "F.Cu") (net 7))
 (segment (start 152.6 46.525) (end 152.475 46.4) (width 0.25) (layer "F.Cu") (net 7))
 (segment (start 157.95 44.225) (end 157.95 46.5) (width 0.25) (layer "F.Cu") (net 3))
 (segment (start 152.654 53.846) (end 152.654 54.4) (width 0.25) (layer "F.Cu") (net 3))
 (segment (start 157.95 47.75) (end 158.1 47.9) (width 0.25) (layer "F.Cu") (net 3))
 (segment (start 154.2 53.1) (end 154.1 53.2) (width 0.25) (layer "F.Cu") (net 3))
 (segment (start 153.3 53.2) (end 152.654 53.846) (width 0.25) (layer "F.Cu") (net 3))
 (segment (start 154.1 53.2) (end 153.3 53.2) (width 0.25) (layer "F.Cu") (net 3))
 (segment (start 157.95 46.5) (end 157.95 47.75) (width 0.25) (layer "F.Cu") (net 3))
 (via (at 158.1 47.9) (size 0.6) (drill 0.4) (layers "F.Cu" "B.Cu") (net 3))
 (via (at 154.2 53.1) (size 0.6) (drill 0.4) (layers "F.Cu" "B.Cu") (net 3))
 (segment (start 158.1 47.9) (end 157.475489 47.275489) (width 0.25) (layer "B.Cu") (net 3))
 (segment (start 154.2 48) (end 154.2 53.1) (width 0.25) (layer "B.Cu") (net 3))
 (segment (start 154.924511 47.275489) (end 154.2 48) (width 0.25) (layer "B.Cu") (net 3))
 (segment (start 157.475489 47.275489) (end 154.924511 47.275489) (width 0.25) (layer "B.Cu") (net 3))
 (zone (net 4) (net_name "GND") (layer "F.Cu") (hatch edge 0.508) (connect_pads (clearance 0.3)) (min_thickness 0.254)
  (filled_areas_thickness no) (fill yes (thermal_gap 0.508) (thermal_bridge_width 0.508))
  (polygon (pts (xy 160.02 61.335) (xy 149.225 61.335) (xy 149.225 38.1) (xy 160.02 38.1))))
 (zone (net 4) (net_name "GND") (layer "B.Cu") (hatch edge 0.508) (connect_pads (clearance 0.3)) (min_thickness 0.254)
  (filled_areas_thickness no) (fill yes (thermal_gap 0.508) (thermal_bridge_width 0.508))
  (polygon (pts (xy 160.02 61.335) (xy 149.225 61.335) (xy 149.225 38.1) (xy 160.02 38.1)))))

